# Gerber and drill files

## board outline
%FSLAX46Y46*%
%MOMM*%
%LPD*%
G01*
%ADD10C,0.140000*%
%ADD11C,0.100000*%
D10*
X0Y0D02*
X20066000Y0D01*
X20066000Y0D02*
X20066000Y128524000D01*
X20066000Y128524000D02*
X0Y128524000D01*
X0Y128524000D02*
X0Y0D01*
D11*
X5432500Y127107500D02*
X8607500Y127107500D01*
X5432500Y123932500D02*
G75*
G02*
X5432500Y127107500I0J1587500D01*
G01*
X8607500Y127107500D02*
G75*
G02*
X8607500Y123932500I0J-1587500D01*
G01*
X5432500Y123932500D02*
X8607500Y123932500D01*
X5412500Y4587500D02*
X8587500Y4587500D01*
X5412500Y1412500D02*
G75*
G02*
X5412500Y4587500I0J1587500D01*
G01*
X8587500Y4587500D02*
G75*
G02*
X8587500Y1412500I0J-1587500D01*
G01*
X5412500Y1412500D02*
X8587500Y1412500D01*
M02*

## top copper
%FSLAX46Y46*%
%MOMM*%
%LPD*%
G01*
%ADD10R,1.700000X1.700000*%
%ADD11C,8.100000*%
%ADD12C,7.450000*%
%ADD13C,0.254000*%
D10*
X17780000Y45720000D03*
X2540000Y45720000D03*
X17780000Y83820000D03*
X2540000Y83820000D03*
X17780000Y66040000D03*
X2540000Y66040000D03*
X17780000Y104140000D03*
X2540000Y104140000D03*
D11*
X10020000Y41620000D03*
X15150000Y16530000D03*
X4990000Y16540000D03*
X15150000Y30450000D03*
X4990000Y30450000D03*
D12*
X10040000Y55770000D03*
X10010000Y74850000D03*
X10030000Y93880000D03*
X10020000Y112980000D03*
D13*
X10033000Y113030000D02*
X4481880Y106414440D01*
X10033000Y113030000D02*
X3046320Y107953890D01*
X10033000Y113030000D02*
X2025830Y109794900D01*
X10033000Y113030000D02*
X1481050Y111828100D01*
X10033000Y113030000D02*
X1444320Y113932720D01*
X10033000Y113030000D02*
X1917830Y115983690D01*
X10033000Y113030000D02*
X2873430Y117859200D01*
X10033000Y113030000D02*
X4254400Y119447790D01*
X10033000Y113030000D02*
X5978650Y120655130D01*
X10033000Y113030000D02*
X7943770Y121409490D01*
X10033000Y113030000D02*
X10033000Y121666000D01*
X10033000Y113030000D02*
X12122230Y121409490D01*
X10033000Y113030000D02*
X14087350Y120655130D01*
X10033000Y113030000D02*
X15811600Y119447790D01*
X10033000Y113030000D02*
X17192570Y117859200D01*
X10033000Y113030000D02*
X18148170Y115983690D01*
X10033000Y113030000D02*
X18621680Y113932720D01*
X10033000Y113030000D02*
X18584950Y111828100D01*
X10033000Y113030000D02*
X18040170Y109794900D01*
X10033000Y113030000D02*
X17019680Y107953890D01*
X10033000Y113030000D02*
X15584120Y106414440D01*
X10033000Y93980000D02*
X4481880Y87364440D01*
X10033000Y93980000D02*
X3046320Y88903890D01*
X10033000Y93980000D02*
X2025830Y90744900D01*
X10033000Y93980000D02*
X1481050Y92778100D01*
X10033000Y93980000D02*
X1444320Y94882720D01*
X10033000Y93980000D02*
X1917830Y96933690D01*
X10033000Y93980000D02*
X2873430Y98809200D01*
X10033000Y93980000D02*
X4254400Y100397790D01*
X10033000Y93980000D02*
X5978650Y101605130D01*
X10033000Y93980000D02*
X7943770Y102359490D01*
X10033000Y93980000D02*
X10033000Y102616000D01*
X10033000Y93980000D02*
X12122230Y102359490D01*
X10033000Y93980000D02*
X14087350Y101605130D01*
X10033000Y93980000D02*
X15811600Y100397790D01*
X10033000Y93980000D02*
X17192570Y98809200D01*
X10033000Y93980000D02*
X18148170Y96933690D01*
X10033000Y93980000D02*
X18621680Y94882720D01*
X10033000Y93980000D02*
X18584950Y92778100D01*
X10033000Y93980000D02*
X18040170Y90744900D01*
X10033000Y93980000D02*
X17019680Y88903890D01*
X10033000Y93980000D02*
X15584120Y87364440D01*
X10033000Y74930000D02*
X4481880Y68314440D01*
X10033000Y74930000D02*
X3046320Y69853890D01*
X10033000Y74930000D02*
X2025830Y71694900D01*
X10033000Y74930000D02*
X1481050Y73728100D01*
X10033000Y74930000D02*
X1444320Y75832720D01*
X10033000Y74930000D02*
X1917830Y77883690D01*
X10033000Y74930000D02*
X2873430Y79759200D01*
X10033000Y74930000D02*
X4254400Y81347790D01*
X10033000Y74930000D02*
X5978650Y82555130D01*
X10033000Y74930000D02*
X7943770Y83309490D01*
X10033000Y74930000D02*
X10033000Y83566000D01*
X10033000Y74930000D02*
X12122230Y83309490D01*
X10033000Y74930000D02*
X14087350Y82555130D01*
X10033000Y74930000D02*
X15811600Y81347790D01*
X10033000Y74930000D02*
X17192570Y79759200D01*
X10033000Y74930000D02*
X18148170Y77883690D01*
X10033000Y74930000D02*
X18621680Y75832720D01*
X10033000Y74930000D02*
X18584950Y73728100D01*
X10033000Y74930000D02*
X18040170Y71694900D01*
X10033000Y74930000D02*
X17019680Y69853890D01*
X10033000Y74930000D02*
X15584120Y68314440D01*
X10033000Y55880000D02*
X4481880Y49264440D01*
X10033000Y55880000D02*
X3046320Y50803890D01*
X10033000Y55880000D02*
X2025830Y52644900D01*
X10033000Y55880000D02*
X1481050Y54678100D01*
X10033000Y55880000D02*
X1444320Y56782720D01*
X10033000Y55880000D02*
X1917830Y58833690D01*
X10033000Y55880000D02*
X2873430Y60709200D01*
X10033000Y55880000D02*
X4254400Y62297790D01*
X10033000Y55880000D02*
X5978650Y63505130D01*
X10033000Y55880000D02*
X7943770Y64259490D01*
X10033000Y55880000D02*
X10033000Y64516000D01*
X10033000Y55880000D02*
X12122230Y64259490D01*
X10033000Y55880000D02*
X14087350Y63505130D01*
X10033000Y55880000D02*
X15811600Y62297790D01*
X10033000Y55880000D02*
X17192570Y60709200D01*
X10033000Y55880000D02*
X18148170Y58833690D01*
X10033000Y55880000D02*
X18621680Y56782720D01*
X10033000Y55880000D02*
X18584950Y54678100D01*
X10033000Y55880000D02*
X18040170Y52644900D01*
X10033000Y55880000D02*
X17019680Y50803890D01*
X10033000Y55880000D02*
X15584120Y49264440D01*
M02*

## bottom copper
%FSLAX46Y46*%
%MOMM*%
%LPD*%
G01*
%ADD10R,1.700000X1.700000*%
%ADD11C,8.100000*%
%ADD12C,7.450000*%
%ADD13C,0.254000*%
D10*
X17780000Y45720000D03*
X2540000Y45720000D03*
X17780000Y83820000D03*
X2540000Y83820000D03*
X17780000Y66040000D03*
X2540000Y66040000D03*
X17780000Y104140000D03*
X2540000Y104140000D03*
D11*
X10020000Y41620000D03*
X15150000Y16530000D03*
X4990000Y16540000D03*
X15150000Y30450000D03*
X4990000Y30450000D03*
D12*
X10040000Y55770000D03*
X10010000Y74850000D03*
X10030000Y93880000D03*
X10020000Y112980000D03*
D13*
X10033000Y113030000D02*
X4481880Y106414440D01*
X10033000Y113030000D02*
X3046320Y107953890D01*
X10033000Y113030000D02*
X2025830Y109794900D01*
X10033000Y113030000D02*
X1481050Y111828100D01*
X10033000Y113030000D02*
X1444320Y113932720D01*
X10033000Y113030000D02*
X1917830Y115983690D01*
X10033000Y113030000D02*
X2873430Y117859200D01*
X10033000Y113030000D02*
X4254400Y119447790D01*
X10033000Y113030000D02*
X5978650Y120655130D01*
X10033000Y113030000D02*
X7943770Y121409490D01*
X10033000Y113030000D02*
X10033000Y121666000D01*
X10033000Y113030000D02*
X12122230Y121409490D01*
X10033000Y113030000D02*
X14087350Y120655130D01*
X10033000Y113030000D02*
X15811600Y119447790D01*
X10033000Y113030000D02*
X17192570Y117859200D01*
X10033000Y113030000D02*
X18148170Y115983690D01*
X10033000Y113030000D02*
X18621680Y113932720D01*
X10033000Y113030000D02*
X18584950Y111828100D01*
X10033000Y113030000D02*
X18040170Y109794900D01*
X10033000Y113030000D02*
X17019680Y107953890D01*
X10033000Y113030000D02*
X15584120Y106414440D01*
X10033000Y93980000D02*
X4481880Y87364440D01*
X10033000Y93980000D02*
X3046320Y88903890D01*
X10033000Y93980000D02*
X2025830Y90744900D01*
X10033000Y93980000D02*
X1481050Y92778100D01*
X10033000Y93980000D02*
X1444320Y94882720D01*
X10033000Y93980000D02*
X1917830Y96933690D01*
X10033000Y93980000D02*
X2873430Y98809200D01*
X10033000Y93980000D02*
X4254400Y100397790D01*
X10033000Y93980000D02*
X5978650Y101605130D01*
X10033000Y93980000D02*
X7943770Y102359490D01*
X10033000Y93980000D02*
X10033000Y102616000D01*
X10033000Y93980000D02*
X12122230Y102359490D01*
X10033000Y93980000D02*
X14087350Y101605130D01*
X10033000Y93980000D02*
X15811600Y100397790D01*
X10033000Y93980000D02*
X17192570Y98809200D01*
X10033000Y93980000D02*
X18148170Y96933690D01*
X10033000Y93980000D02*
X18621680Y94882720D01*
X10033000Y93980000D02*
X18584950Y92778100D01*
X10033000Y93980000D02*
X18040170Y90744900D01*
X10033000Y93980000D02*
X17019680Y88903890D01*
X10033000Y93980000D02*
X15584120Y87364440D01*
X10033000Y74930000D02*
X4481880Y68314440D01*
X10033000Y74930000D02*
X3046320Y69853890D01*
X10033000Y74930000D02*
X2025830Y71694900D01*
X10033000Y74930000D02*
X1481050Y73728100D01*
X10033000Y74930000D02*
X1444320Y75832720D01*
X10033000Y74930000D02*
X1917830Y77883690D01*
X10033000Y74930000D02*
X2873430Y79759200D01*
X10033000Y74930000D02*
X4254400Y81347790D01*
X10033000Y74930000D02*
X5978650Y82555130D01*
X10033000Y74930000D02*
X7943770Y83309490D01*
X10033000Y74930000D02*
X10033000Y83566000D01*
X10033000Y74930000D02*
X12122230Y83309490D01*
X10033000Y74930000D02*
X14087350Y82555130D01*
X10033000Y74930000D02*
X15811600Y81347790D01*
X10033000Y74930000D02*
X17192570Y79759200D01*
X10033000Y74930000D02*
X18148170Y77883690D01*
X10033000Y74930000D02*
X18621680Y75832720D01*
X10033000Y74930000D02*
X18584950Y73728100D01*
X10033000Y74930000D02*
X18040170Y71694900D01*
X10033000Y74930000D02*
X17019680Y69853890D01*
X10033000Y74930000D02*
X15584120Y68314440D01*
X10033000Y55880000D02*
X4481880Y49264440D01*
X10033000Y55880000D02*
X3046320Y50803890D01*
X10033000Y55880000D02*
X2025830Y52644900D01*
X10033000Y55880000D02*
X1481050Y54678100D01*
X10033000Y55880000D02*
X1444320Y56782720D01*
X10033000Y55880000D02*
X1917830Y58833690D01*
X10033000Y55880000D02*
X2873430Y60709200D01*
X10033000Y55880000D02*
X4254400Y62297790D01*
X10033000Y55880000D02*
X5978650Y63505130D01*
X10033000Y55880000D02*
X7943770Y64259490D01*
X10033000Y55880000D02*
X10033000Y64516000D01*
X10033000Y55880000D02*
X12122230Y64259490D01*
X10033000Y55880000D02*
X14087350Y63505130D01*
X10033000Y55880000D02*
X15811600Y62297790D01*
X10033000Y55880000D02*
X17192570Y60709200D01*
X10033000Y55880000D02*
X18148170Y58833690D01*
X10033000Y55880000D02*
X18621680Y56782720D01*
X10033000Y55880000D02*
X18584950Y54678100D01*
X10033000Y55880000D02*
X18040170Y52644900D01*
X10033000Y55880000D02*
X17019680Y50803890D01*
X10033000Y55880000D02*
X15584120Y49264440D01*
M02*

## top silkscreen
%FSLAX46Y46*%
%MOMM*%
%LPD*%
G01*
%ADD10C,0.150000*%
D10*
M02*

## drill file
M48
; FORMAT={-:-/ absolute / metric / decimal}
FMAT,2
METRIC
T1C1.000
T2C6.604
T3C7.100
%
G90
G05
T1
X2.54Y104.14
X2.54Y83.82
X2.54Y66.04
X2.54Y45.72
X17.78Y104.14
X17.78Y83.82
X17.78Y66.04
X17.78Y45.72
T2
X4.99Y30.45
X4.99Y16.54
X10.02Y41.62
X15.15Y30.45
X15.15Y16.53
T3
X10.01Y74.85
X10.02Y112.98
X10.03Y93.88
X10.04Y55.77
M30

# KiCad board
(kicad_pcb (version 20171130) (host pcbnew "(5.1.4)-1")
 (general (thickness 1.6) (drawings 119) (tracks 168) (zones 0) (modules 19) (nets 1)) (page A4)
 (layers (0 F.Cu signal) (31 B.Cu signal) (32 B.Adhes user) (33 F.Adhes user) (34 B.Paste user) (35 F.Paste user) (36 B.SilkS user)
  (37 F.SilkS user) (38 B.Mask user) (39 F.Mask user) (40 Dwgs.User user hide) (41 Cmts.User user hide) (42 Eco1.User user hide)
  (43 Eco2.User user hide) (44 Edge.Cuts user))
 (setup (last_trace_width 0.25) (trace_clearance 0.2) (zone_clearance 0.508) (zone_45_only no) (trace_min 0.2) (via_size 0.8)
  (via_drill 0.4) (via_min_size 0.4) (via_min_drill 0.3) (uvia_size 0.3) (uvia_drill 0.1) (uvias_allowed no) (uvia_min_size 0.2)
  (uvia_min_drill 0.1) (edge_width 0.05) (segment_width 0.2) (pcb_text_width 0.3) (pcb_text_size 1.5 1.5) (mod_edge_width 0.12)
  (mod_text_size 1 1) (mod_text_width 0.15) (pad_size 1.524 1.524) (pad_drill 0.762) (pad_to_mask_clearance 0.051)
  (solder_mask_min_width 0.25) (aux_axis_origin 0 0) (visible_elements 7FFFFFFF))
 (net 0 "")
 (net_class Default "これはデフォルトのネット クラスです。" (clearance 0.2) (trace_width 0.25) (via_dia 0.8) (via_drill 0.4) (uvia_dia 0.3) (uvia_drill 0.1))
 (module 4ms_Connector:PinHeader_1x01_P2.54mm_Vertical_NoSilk (layer F.Cu) (at 17.78 -45.72)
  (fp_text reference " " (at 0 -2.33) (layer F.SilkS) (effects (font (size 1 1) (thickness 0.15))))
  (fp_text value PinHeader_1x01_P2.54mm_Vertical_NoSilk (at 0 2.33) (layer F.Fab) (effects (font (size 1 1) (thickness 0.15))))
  (pad 1 thru_hole rect (at 0 0) (size 1.7 1.7) (drill 1) (layers *.Cu *.Mask)))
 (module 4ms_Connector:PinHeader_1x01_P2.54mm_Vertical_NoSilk (layer F.Cu) (at 2.54 -45.72)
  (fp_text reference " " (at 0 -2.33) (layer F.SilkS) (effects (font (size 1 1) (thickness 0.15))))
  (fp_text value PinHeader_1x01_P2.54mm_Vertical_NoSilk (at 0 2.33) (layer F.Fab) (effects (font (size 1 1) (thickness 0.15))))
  (pad 1 thru_hole rect (at 0 0) (size 1.7 1.7) (drill 1) (layers *.Cu *.Mask)))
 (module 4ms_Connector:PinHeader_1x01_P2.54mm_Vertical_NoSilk (layer F.Cu) (at 17.78 -83.82)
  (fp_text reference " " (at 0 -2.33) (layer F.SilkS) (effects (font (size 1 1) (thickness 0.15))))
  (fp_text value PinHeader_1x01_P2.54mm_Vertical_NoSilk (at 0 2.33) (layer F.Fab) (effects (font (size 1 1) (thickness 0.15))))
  (pad 1 thru_hole rect (at 0 0) (size 1.7 1.7) (drill 1) (layers *.Cu *.Mask)))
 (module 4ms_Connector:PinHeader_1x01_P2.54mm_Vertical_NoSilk (layer F.Cu) (at 2.54 -83.82)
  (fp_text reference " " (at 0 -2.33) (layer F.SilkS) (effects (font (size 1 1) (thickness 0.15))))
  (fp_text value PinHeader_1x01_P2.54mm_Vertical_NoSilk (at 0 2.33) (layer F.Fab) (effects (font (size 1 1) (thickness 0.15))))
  (pad 1 thru_hole rect (at 0 0) (size 1.7 1.7) (drill 1) (layers *.Cu *.Mask)))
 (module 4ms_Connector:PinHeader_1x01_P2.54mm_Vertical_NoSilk (layer F.Cu) (at 17.78 -66.04)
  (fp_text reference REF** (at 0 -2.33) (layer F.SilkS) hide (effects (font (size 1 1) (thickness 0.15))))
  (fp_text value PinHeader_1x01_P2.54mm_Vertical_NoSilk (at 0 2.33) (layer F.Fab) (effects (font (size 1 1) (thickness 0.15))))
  (pad 1 thru_hole rect (at 0 0) (size 1.7 1.7) (drill 1) (layers *.Cu *.Mask)))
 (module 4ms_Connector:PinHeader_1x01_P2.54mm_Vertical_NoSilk (layer F.Cu) (at 2.54 -66.04)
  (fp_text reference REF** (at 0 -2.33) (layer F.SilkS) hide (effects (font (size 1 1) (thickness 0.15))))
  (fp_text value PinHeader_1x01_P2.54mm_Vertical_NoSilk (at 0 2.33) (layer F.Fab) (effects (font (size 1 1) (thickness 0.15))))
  (pad 1 thru_hole rect (at 0 0) (size 1.7 1.7) (drill 1) (layers *.Cu *.Mask)))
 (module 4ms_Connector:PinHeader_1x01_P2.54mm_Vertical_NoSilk (layer F.Cu) (at 17.78 -104.14)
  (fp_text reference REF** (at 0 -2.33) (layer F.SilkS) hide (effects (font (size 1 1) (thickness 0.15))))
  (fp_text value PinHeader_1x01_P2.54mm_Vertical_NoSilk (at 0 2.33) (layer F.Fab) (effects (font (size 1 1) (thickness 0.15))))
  (pad 1 thru_hole rect (at 0 0) (size 1.7 1.7) (drill 1) (layers *.Cu *.Mask)))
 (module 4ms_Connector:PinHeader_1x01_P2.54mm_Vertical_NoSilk (layer F.Cu) (at 2.54 -104.14)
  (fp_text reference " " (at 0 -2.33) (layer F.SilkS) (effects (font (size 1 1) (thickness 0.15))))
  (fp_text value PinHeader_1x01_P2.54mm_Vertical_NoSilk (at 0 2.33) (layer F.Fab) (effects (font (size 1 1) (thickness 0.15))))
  (pad 1 thru_hole rect (at 0 0) (size 1.7 1.7) (drill 1) (layers *.Cu *.Mask)))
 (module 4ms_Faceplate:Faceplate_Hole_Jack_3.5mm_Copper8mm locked (layer F.Cu) (at 10.02 -41.62)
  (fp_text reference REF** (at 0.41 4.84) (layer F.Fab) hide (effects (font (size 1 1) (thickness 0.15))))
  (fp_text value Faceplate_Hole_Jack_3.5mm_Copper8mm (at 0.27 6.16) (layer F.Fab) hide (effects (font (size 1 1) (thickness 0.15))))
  (pad 1 thru_hole circle (at 0 0) (size 8.1 8.1) (drill 6.604) (layers *.Cu *.Mask)))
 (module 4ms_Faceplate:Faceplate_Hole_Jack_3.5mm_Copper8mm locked (layer F.Cu) (at 15.15 -16.53)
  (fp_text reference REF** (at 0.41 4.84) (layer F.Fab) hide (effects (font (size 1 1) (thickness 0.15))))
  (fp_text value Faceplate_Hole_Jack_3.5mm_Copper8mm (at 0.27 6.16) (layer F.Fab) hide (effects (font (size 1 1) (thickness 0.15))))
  (pad 1 thru_hole circle (at 0 0) (size 8.1 8.1) (drill 6.604) (layers *.Cu *.Mask)))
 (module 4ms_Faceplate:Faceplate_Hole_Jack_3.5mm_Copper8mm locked (layer F.Cu) (at 4.99 -16.54)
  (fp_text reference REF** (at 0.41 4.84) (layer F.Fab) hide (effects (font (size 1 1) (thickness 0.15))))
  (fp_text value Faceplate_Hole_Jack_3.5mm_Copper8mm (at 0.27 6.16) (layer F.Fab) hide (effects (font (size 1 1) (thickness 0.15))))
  (pad 1 thru_hole circle (at 0 0) (size 8.1 8.1) (drill 6.604) (layers *.Cu *.Mask)))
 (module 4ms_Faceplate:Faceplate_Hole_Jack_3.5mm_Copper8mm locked (layer F.Cu) (at 15.15 -30.45)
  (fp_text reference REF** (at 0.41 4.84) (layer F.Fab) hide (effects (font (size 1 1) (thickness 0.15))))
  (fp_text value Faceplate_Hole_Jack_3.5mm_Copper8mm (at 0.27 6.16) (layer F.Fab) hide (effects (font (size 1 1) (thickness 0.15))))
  (pad 1 thru_hole circle (at 0 0) (size 8.1 8.1) (drill 6.604) (layers *.Cu *.Mask)))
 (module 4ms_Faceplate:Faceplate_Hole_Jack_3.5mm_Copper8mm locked (layer F.Cu) (at 4.99 -30.45)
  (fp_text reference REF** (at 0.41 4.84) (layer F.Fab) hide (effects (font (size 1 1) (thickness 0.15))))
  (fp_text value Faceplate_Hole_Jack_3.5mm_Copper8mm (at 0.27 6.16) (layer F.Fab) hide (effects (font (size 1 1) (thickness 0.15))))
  (pad 1 thru_hole circle (at 0 0) (size 8.1 8.1) (drill 6.604) (layers *.Cu *.Mask)))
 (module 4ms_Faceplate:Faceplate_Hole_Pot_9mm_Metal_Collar (layer F.Cu) (at 10.04 -55.77)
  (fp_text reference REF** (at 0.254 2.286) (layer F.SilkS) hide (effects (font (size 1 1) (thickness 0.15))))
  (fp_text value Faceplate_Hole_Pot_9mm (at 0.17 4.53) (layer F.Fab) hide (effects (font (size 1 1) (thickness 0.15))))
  (pad 1 thru_hole circle (at 0 0) (size 7.45 7.45) (drill 7.1) (layers *.Cu *.Mask)))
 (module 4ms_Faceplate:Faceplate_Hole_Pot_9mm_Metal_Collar (layer F.Cu) (at 10.01 -74.85)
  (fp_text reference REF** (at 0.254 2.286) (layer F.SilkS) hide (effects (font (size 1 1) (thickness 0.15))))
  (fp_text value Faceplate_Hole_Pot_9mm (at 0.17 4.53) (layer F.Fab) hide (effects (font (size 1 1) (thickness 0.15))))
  (pad 1 thru_hole circle (at 0 0) (size 7.45 7.45) (drill 7.1) (layers *.Cu *.Mask)))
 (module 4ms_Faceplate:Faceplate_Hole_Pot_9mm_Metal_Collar (layer F.Cu) (at 10.03 -93.88)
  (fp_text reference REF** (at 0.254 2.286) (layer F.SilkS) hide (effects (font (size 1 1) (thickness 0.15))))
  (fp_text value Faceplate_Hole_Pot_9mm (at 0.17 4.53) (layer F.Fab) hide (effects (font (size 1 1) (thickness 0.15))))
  (pad 1 thru_hole circle (at 0 0) (size 7.45 7.45) (drill 7.1) (layers *.Cu *.Mask)))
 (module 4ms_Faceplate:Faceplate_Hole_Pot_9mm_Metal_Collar (layer F.Cu) (at 10.02 -112.98)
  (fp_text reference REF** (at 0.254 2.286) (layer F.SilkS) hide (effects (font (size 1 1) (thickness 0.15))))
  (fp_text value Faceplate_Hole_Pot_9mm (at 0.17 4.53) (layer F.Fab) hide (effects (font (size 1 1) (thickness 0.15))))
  (pad 1 thru_hole circle (at 0 0) (size 7.45 7.45) (drill 7.1) (layers *.Cu *.Mask)))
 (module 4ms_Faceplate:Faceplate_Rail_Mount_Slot (layer F.Cu) (at 7.02 -125.52)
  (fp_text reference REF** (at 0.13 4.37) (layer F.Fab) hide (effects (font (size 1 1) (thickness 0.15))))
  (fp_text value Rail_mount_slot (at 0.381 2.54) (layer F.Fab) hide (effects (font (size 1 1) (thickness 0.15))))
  (fp_line (start -1.5875 -1.5875) (end 1.5875 -1.5875) (layer Edge.Cuts) (width 0.1))
  (fp_arc (start -1.5875 0) (end -1.5875 1.5875) (angle 180) (layer Edge.Cuts) (width 0.1))
  (fp_arc (start 1.5875 0) (end 1.5875 -1.5875) (angle 180) (layer Edge.Cuts) (width 0.1))
  (fp_line (start -1.5875 1.5875) (end 1.5875 1.5875) (layer Edge.Cuts) (width 0.1)))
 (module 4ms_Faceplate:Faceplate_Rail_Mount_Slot (layer F.Cu) (at 7 -3)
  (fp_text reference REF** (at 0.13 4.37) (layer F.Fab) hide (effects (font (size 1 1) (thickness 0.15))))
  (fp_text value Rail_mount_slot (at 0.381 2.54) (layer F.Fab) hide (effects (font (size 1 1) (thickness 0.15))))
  (fp_line (start -1.5875 -1.5875) (end 1.5875 -1.5875) (layer Edge.Cuts) (width 0.1))
  (fp_arc (start -1.5875 0) (end -1.5875 1.5875) (angle 180) (layer Edge.Cuts) (width 0.1))
  (fp_arc (start 1.5875 0) (end 1.5875 -1.5875) (angle 180) (layer Edge.Cuts) (width 0.1))
  (fp_line (start -1.5875 1.5875) (end 1.5875 1.5875) (layer Edge.Cuts) (width 0.1)))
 (gr_line (start 0 0) (end 20.066 0) (layer Edge.Cuts) (width 0.14))
 (gr_line (start 20.066 0) (end 20.066 -128.524) (layer Edge.Cuts) (width 0.14))
 (gr_line (start 20.066 -128.524) (end 0 -128.524) (layer Edge.Cuts) (width 0.14))
 (gr_line (start 0 -128.524) (end 0 0) (layer Edge.Cuts) (width 0.14))
 (segment (start 10.033 -113.03) (end 4.48188 -106.41444) (width 0.254) (layer B.Cu) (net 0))
 (segment (start 10.033 -113.03) (end 3.04632 -107.95389) (width 0.254) (layer B.Cu) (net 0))
 (segment (start 10.033 -113.03) (end 2.02583 -109.7949) (width 0.254) (layer B.Cu) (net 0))
 (segment (start 10.033 -113.03) (end 1.48105 -111.8281) (width 0.254) (layer B.Cu) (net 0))
 (segment (start 10.033 -113.03) (end 1.44432 -113.93272) (width 0.254) (layer B.Cu) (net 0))
 (segment (start 10.033 -113.03) (end 1.91783 -115.98369) (width 0.254) (layer B.Cu) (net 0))
 (segment (start 10.033 -113.03) (end 2.87343 -117.8592) (width 0.254) (layer B.Cu) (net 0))
 (segment (start 10.033 -113.03) (end 4.2544 -119.44779) (width 0.254) (layer B.Cu) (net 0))
 (segment (start 10.033 -113.03) (end 5.97865 -120.65513) (width 0.254) (layer B.Cu) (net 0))
 (segment (start 10.033 -113.03) (end 7.94377 -121.40949) (width 0.254) (layer B.Cu) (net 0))
 (segment (start 10.033 -113.03) (end 10.033 -121.666) (width 0.254) (layer B.Cu) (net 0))
 (segment (start 10.033 -113.03) (end 12.12223 -121.40949) (width 0.254) (layer B.Cu) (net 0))
 (segment (start 10.033 -113.03) (end 14.08735 -120.65513) (width 0.254) (layer B.Cu) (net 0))
 (segment (start 10.033 -113.03) (end 15.8116 -119.44779) (width 0.254) (layer B.Cu) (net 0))
 (segment (start 10.033 -113.03) (end 17.19257 -117.8592) (width 0.254) (layer B.Cu) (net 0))
 (segment (start 10.033 -113.03) (end 18.14817 -115.98369) (width 0.254) (layer B.Cu) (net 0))
 (segment (start 10.033 -113.03) (end 18.62168 -113.93272) (width 0.254) (layer B.Cu) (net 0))
 (segment (start 10.033 -113.03) (end 18.58495 -111.8281) (width 0.254) (layer B.Cu) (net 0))
 (segment (start 10.033 -113.03) (end 18.04017 -109.7949) (width 0.254) (layer B.Cu) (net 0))
 (segment (start 10.033 -113.03) (end 17.01968 -107.95389) (width 0.254) (layer B.Cu) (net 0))
 (segment (start 10.033 -113.03) (end 15.58412 -106.41444) (width 0.254) (layer B.Cu) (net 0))
 (segment (start 10.033 -93.98) (end 4.48188 -87.36444) (width 0.254) (layer B.Cu) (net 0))
 (segment (start 10.033 -93.98) (end 3.04632 -88.90389) (width 0.254) (layer B.Cu) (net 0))
 (segment (start 10.033 -93.98) (end 2.02583 -90.7449) (width 0.254) (layer B.Cu) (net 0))
 (segment (start 10.033 -93.98) (end 1.48105 -92.7781) (width 0.254) (layer B.Cu) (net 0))
 (segment (start 10.033 -93.98) (end 1.44432 -94.88272) (width 0.254) (layer B.Cu) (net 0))
 (segment (start 10.033 -93.98) (end 1.91783 -96.93369) (width 0.254) (layer B.Cu) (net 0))
 (segment (start 10.033 -93.98) (end 2.87343 -98.8092) (width 0.254) (layer B.Cu) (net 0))
 (segment (start 10.033 -93.98) (end 4.2544 -100.39779) (width 0.254) (layer B.Cu) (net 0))
 (segment (start 10.033 -93.98) (end 5.97865 -101.60513) (width 0.254) (layer B.Cu) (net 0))
 (segment (start 10.033 -93.98) (end 7.94377 -102.35949) (width 0.254) (layer B.Cu) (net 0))
 (segment (start 10.033 -93.98) (end 10.033 -102.616) (width 0.254) (layer B.Cu) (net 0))
 (segment (start 10.033 -93.98) (end 12.12223 -102.35949) (width 0.254) (layer B.Cu) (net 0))
 (segment (start 10.033 -93.98) (end 14.08735 -101.60513) (width 0.254) (layer B.Cu) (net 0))
 (segment (start 10.033 -93.98) (end 15.8116 -100.39779) (width 0.254) (layer B.Cu) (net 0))
 (segment (start 10.033 -93.98) (end 17.19257 -98.8092) (width 0.254) (layer B.Cu) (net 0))
 (segment (start 10.033 -93.98) (end 18.14817 -96.93369) (width 0.254) (layer B.Cu) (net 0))
 (segment (start 10.033 -93.98) (end 18.62168 -94.88272) (width 0.254) (layer B.Cu) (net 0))
 (segment (start 10.033 -93.98) (end 18.58495 -92.7781) (width 0.254) (layer B.Cu) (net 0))
 (segment (start 10.033 -93.98) (end 18.04017 -90.7449) (width 0.254) (layer B.Cu) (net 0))
 (segment (start 10.033 -93.98) (end 17.01968 -88.90389) (width 0.254) (layer B.Cu) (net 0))
 (segment (start 10.033 -93.98) (end 15.58412 -87.36444) (width 0.254) (layer B.Cu) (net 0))
 (segment (start 10.033 -74.93) (end 4.48188 -68.31444) (width 0.254) (layer B.Cu) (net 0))
 (segment (start 10.033 -74.93) (end 3.04632 -69.85389) (width 0.254) (layer B.Cu) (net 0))
 (segment (start 10.033 -74.93) (end 2.02583 -71.6949) (width 0.254) (layer B.Cu) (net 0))
 (segment (start 10.033 -74.93) (end 1.48105 -73.7281) (width 0.254) (layer B.Cu) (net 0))
 (segment (start 10.033 -74.93) (end 1.44432 -75.83272) (width 0.254) (layer B.Cu) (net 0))
 (segment (start 10.033 -74.93) (end 1.91783 -77.88369) (width 0.254) (layer B.Cu) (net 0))
 (segment (start 10.033 -74.93) (end 2.87343 -79.7592) (width 0.254) (layer B.Cu) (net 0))
 (segment (start 10.033 -74.93) (end 4.2544 -81.34779) (width 0.254) (layer B.Cu) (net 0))
 (segment (start 10.033 -74.93) (end 5.97865 -82.55513) (width 0.254) (layer B.Cu) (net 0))
 (segment (start 10.033 -74.93) (end 7.94377 -83.30949) (width 0.254) (layer B.Cu) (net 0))
 (segment (start 10.033 -74.93) (end 10.033 -83.566) (width 0.254) (layer B.Cu) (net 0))
 (segment (start 10.033 -74.93) (end 12.12223 -83.30949) (width 0.254) (layer B.Cu) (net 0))
 (segment (start 10.033 -74.93) (end 14.08735 -82.55513) (width 0.254) (layer B.Cu) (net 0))
 (segment (start 10.033 -74.93) (end 15.8116 -81.34779) (width 0.254) (layer B.Cu) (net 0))
 (segment (start 10.033 -74.93) (end 17.19257 -79.7592) (width 0.254) (layer B.Cu) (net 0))
 (segment (start 10.033 -74.93) (end 18.14817 -77.88369) (width 0.254) (layer B.Cu) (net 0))
 (segment (start 10.033 -74.93) (end 18.62168 -75.83272) (width 0.254) (layer B.Cu) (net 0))
 (segment (start 10.033 -74.93) (end 18.58495 -73.7281) (width 0.254) (layer B.Cu) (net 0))
 (segment (start 10.033 -74.93) (end 18.04017 -71.6949) (width 0.254) (layer B.Cu) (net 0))
 (segment (start 10.033 -74.93) (end 17.01968 -69.85389) (width 0.254) (layer B.Cu) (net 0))
 (segment (start 10.033 -74.93) (end 15.58412 -68.31444) (width 0.254) (layer B.Cu) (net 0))
 (segment (start 10.033 -55.88) (end 4.48188 -49.26444) (width 0.254) (layer B.Cu) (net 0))
 (segment (start 10.033 -55.88) (end 3.04632 -50.80389) (width 0.254) (layer B.Cu) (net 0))
 (segment (start 10.033 -55.88) (end 2.02583 -52.6449) (width 0.254) (layer B.Cu) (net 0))
 (segment (start 10.033 -55.88) (end 1.48105 -54.6781) (width 0.254) (layer B.Cu) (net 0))
 (segment (start 10.033 -55.88) (end 1.44432 -56.78272) (width 0.254) (layer B.Cu) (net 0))
 (segment (start 10.033 -55.88) (end 1.91783 -58.83369) (width 0.254) (layer B.Cu) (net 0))
 (segment (start 10.033 -55.88) (end 2.87343 -60.7092) (width 0.254) (layer B.Cu) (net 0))
 (segment (start 10.033 -55.88) (end 4.2544 -62.29779) (width 0.254) (layer B.Cu) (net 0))
 (segment (start 10.033 -55.88) (end 5.97865 -63.50513) (width 0.254) (layer B.Cu) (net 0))
 (segment (start 10.033 -55.88) (end 7.94377 -64.25949) (width 0.254) (layer B.Cu) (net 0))
 (segment (start 10.033 -55.88) (end 10.033 -64.516) (width 0.254) (layer B.Cu) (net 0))
 (segment (start 10.033 -55.88) (end 12.12223 -64.25949) (width 0.254) (layer B.Cu) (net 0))
 (segment (start 10.033 -55.88) (end 14.08735 -63.50513) (width 0.254) (layer B.Cu) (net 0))
 (segment (start 10.033 -55.88) (end 15.8116 -62.29779) (width 0.254) (layer B.Cu) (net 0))
 (segment (start 10.033 -55.88) (end 17.19257 -60.7092) (width 0.254) (layer B.Cu) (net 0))
 (segment (start 10.033 -55.88) (end 18.14817 -58.83369) (width 0.254) (layer B.Cu) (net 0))
 (segment (start 10.033 -55.88) (end 18.62168 -56.78272) (width 0.254) (layer B.Cu) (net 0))
 (segment (start 10.033 -55.88) (end 18.58495 -54.6781) (width 0.254) (layer B.Cu) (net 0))
 (segment (start 10.033 -55.88) (end 18.04017 -52.6449) (width 0.254) (layer B.Cu) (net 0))
 (segment (start 10.033 -55.88) (end 17.01968 -50.80389) (width 0.254) (layer B.Cu) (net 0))
 (segment (start 10.033 -55.88) (end 15.58412 -49.26444) (width 0.254) (layer B.Cu) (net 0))
 (segment (start 10.033 -113.03) (end 4.48188 -106.41444) (width 0.254) (layer F.Cu) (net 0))
 (segment (start 10.033 -113.03) (end 3.04632 -107.95389) (width 0.254) (layer F.Cu) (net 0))
 (segment (start 10.033 -113.03) (end 2.02583 -109.7949) (width 0.254) (layer F.Cu) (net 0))
 (segment (start 10.033 -113.03) (end 1.48105 -111.8281) (width 0.254) (layer F.Cu) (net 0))
 (segment (start 10.033 -113.03) (end 1.44432 -113.93272) (width 0.254) (layer F.Cu) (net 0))
 (segment (start 10.033 -113.03) (end 1.91783 -115.98369) (width 0.254) (layer F.Cu) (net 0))
 (segment (start 10.033 -113.03) (end 2.87343 -117.8592) (width 0.254) (layer F.Cu) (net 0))
 (segment (start 10.033 -113.03) (end 4.2544 -119.44779) (width 0.254) (layer F.Cu) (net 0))
 (segment (start 10.033 -113.03) (end 5.97865 -120.65513) (width 0.254) (layer F.Cu) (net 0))
 (segment (start 10.033 -113.03) (end 7.94377 -121.40949) (width 0.254) (layer F.Cu) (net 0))
 (segment (start 10.033 -113.03) (end 10.033 -121.666) (width 0.254) (layer F.Cu) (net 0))
 (segment (start 10.033 -113.03) (end 12.12223 -121.40949) (width 0.254) (layer F.Cu) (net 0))
 (segment (start 10.033 -113.03) (end 14.08735 -120.65513) (width 0.254) (layer F.Cu) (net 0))
 (segment (start 10.033 -113.03) (end 15.8116 -119.44779) (width 0.254) (layer F.Cu) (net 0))
 (segment (start 10.033 -113.03) (end 17.19257 -117.8592) (width 0.254) (layer F.Cu) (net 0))
 (segment (start 10.033 -113.03) (end 18.14817 -115.98369) (width 0.254) (layer F.Cu) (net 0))
 (segment (start 10.033 -113.03) (end 18.62168 -113.93272) (width 0.254) (layer F.Cu) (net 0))
 (segment (start 10.033 -113.03) (end 18.58495 -111.8281) (width 0.254) (layer F.Cu) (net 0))
 (segment (start 10.033 -113.03) (end 18.04017 -109.7949) (width 0.254) (layer F.Cu) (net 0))
 (segment (start 10.033 -113.03) (end 17.01968 -107.95389) (width 0.254) (layer F.Cu) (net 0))
 (segment (start 10.033 -113.03) (end 15.58412 -106.41444) (width 0.254) (layer F.Cu) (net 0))
 (segment (start 10.033 -93.98) (end 4.48188 -87.36444) (width 0.254) (layer F.Cu) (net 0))
 (segment (start 10.033 -93.98) (end 3.04632 -88.90389) (width 0.254) (layer F.Cu) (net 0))
 (segment (start 10.033 -93.98) (end 2.02583 -90.7449) (width 0.254) (layer F.Cu) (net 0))
 (segment (start 10.033 -93.98) (end 1.48105 -92.7781) (width 0.254) (layer F.Cu) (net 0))
 (segment (start 10.033 -93.98) (end 1.44432 -94.88272) (width 0.254) (layer F.Cu) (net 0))
 (segment (start 10.033 -93.98) (end 1.91783 -96.93369) (width 0.254) (layer F.Cu) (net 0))
 (segment (start 10.033 -93.98) (end 2.87343 -98.8092) (width 0.254) (layer F.Cu) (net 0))
 (segment (start 10.033 -93.98) (end 4.2544 -100.39779) (width 0.254) (layer F.Cu) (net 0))
 (segment (start 10.033 -93.98) (end 5.97865 -101.60513) (width 0.254) (layer F.Cu) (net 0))
 (segment (start 10.033 -93.98) (end 7.94377 -102.35949) (width 0.254) (layer F.Cu) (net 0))
 (segment (start 10.033 -93.98) (end 10.033 -102.616) (width 0.254) (layer F.Cu) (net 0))
 (segment (start 10.033 -93.98) (end 12.12223 -102.35949) (width 0.254) (layer F.Cu) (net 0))
 (segment (start 10.033 -93.98) (end 14.08735 -101.60513) (width 0.254) (layer F.Cu) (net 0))
 (segment (start 10.033 -93.98) (end 15.8116 -100.39779) (width 0.254) (layer F.Cu) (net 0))
 (segment (start 10.033 -93.98) (end 17.19257 -98.8092) (width 0.254) (layer F.Cu) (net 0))
 (segment (start 10.033 -93.98) (end 18.14817 -96.93369) (width 0.254) (layer F.Cu) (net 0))
 (segment (start 10.033 -93.98) (end 18.62168 -94.88272) (width 0.254) (layer F.Cu) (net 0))
 (segment (start 10.033 -93.98) (end 18.58495 -92.7781) (width 0.254) (layer F.Cu) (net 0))
 (segment (start 10.033 -93.98) (end 18.04017 -90.7449) (width 0.254) (layer F.Cu) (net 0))
 (segment (start 10.033 -93.98) (end 17.01968 -88.90389) (width 0.254) (layer F.Cu) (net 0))
 (segment (start 10.033 -93.98) (end 15.58412 -87.36444) (width 0.254) (layer F.Cu) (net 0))
 (segment (start 10.033 -74.93) (end 4.48188 -68.31444) (width 0.254) (layer F.Cu) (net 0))
 (segment (start 10.033 -74.93) (end 3.04632 -69.85389) (width 0.254) (layer F.Cu) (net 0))
 (segment (start 10.033 -74.93) (end 2.02583 -71.6949) (width 0.254) (layer F.Cu) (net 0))
 (segment (start 10.033 -74.93) (end 1.48105 -73.7281) (width 0.254) (layer F.Cu) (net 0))
 (segment (start 10.033 -74.93) (end 1.44432 -75.83272) (width 0.254) (layer F.Cu) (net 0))
 (segment (start 10.033 -74.93) (end 1.91783 -77.88369) (width 0.254) (layer F.Cu) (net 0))
 (segment (start 10.033 -74.93) (end 2.87343 -79.7592) (width 0.254) (layer F.Cu) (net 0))
 (segment (start 10.033 -74.93) (end 4.2544 -81.34779) (width 0.254) (layer F.Cu) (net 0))
 (segment (start 10.033 -74.93) (end 5.97865 -82.55513) (width 0.254) (layer F.Cu) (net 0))
 (segment (start 10.033 -74.93) (end 7.94377 -83.30949) (width 0.254) (layer F.Cu) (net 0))
 (segment (start 10.033 -74.93) (end 10.033 -83.566) (width 0.254) (layer F.Cu) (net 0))
 (segment (start 10.033 -74.93) (end 12.12223 -83.30949) (width 0.254) (layer F.Cu) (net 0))
 (segment (start 10.033 -74.93) (end 14.08735 -82.55513) (width 0.254) (layer F.Cu) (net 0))
 (segment (start 10.033 -74.93) (end 15.8116 -81.34779) (width 0.254) (layer F.Cu) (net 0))
 (segment (start 10.033 -74.93) (end 17.19257 -79.7592) (width 0.254) (layer F.Cu) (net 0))
 (segment (start 10.033 -74.93) (end 18.14817 -77.88369) (width 0.254) (layer F.Cu) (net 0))
 (segment (start 10.033 -74.93) (end 18.62168 -75.83272) (width 0.254) (layer F.Cu) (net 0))
 (segment (start 10.033 -74.93) (end 18.58495 -73.7281) (width 0.254) (layer F.Cu) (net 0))
 (segment (start 10.033 -74.93) (end 18.04017 -71.6949) (width 0.254) (layer F.Cu) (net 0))
 (segment (start 10.033 -74.93) (end 17.01968 -69.85389) (width 0.254) (layer F.Cu) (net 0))
 (segment (start 10.033 -74.93) (end 15.58412 -68.31444) (width 0.254) (layer F.Cu) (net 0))
 (segment (start 10.033 -55.88) (end 4.48188 -49.26444) (width 0.254) (layer F.Cu) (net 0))
 (segment (start 10.033 -55.88) (end 3.04632 -50.80389) (width 0.254) (layer F.Cu) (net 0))
 (segment (start 10.033 -55.88) (end 2.02583 -52.6449) (width 0.254) (layer F.Cu) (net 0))
 (segment (start 10.033 -55.88) (end 1.48105 -54.6781) (width 0.254) (layer F.Cu) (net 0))
 (segment (start 10.033 -55.88) (end 1.44432 -56.78272) (width 0.254) (layer F.Cu) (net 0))
 (segment (start 10.033 -55.88) (end 1.91783 -58.83369) (width 0.254) (layer F.Cu) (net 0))
 (segment (start 10.033 -55.88) (end 2.87343 -60.7092) (width 0.254) (layer F.Cu) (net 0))
 (segment (start 10.033 -55.88) (end 4.2544 -62.29779) (width 0.254) (layer F.Cu) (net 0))
 (segment (start 10.033 -55.88) (end 5.97865 -63.50513) (width 0.254) (layer F.Cu) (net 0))
 (segment (start 10.033 -55.88) (end 7.94377 -64.25949) (width 0.254) (layer F.Cu) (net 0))
 (segment (start 10.033 -55.88) (end 10.033 -64.516) (width 0.254) (layer F.Cu) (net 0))
 (segment (start 10.033 -55.88) (end 12.12223 -64.25949) (width 0.254) (layer F.Cu) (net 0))
 (segment (start 10.033 -55.88) (end 14.08735 -63.50513) (width 0.254) (layer F.Cu) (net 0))
 (segment (start 10.033 -55.88) (end 15.8116 -62.29779) (width 0.254) (layer F.Cu) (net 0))
 (segment (start 10.033 -55.88) (end 17.19257 -60.7092) (width 0.254) (layer F.Cu) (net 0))
 (segment (start 10.033 -55.88) (end 18.14817 -58.83369) (width 0.254) (layer F.Cu) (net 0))
 (segment (start 10.033 -55.88) (end 18.62168 -56.78272) (width 0.254) (layer F.Cu) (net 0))
 (segment (start 10.033 -55.88) (end 18.58495 -54.6781) (width 0.254) (layer F.Cu) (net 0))
 (segment (start 10.033 -55.88) (end 18.04017 -52.6449) (width 0.254) (layer F.Cu) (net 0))
 (segment (start 10.033 -55.88) (end 17.01968 -50.80389) (width 0.254) (layer F.Cu) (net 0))
 (segment (start 10.033 -55.88) (end 15.58412 -49.26444) (width 0.254) (layer F.Cu) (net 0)))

